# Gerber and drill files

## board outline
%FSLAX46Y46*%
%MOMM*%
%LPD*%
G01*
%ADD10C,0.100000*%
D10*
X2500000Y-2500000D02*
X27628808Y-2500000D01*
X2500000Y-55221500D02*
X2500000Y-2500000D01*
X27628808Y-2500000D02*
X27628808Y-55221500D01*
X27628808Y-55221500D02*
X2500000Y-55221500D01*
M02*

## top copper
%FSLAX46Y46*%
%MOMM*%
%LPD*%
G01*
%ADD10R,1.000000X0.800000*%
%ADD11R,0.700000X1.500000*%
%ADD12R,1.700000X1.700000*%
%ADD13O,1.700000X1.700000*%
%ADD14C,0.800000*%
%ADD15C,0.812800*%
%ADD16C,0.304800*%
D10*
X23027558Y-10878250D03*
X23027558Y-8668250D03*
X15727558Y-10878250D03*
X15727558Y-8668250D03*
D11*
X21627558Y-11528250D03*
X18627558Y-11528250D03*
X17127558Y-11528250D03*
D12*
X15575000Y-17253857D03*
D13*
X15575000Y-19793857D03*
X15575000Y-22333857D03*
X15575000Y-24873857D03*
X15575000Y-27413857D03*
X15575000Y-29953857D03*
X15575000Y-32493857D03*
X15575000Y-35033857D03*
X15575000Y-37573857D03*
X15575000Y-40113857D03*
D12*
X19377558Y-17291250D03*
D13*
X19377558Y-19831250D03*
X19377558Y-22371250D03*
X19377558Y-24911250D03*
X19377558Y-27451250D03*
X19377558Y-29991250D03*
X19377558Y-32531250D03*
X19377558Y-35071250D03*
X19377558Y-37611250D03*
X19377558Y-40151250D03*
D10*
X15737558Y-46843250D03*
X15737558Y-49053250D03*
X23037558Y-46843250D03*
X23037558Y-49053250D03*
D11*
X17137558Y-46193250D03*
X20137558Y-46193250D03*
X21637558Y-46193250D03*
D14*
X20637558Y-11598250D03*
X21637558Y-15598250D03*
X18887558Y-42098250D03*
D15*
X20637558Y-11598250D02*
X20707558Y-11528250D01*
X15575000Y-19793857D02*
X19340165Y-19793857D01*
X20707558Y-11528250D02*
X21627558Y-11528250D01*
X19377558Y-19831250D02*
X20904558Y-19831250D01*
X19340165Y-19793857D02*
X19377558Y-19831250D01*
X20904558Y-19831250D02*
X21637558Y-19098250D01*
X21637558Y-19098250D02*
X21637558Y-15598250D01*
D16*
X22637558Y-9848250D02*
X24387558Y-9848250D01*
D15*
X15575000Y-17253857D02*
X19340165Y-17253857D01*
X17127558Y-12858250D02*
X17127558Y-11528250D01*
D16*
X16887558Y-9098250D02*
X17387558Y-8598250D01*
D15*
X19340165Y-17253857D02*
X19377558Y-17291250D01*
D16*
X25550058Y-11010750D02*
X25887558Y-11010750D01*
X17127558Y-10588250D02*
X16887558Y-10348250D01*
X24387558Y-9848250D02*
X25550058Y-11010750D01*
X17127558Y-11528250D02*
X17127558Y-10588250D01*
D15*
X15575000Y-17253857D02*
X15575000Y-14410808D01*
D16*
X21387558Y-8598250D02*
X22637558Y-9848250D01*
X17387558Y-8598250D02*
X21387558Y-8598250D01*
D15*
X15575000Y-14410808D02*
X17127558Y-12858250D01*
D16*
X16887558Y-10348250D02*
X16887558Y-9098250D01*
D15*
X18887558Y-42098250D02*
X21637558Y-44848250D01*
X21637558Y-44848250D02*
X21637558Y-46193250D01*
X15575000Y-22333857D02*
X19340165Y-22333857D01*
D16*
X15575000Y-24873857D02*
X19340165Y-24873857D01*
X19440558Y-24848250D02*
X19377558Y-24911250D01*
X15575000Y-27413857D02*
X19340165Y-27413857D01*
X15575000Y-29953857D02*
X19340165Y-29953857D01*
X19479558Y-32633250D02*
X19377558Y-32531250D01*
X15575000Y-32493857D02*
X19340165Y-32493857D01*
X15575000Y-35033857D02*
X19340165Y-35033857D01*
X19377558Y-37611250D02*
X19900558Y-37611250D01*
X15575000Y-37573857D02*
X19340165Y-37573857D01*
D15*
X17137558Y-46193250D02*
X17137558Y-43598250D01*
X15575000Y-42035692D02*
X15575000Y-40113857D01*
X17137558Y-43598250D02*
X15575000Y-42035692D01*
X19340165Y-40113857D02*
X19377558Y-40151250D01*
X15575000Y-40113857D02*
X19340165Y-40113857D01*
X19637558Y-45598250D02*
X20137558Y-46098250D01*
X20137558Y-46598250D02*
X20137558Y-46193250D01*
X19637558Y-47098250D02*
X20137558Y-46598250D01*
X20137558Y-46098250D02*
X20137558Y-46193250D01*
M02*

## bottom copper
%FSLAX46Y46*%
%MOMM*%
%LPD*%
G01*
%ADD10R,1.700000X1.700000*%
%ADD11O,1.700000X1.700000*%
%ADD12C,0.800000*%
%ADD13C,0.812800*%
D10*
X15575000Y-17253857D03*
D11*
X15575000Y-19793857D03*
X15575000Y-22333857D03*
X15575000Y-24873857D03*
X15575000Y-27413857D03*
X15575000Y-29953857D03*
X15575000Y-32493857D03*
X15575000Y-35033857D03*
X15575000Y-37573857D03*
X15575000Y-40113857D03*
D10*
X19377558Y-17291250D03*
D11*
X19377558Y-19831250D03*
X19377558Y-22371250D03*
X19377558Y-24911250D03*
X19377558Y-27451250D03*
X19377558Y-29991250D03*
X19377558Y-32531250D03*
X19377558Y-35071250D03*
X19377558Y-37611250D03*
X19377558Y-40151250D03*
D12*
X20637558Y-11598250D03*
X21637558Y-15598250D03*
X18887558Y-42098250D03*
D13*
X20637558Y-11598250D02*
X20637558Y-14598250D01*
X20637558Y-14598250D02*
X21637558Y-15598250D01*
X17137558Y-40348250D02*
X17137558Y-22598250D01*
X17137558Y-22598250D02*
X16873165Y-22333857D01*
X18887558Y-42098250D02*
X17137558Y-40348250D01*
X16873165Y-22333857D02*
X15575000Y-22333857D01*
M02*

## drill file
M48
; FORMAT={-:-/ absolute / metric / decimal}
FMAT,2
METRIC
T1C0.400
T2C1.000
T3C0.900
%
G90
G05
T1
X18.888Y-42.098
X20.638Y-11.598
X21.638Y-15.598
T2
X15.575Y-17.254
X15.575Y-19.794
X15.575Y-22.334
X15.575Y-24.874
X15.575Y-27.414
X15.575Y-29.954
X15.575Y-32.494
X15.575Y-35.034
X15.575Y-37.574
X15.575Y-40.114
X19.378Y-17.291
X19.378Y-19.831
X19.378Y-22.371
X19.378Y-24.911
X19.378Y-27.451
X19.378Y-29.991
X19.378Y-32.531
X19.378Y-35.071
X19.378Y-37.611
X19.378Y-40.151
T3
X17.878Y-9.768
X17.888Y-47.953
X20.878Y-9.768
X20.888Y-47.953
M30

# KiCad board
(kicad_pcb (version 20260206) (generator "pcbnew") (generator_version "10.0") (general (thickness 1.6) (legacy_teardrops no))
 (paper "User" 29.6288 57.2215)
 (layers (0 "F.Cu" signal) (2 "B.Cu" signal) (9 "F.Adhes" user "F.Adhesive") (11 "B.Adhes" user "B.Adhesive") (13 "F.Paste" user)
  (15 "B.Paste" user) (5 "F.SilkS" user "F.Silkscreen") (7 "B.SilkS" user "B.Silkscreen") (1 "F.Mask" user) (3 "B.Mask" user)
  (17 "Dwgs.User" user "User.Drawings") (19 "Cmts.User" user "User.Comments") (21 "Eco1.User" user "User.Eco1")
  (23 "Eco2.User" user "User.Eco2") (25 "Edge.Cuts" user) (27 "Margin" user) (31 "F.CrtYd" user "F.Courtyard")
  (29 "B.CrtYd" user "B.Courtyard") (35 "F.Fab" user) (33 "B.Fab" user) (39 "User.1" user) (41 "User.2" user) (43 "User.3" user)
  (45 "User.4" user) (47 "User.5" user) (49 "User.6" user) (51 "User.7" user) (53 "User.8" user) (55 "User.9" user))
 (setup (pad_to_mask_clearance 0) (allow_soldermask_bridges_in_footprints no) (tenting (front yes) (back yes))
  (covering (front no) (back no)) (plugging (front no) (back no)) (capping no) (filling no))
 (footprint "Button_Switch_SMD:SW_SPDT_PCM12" (layer "F.Cu") (at 19.377558 10.09825 180)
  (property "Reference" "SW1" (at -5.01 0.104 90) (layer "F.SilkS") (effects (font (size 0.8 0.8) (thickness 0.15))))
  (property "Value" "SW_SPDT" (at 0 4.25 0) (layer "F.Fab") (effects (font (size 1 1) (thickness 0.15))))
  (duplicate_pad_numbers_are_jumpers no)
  (pad "" smd rect (at -3.65 -0.78 180) (size 1 0.8) (layers "F.Cu" "F.Mask" "F.Paste"))
  (pad "" smd rect (at -3.65 1.43 180) (size 1 0.8) (layers "F.Cu" "F.Mask" "F.Paste"))
  (pad "" np_thru_hole circle (at -1.5 0.33 180) (size 0.9 0.9) (drill 0.9) (layers "*.Cu" "*.Mask"))
  (pad "" np_thru_hole circle (at 1.5 0.33 180) (size 0.9 0.9) (drill 0.9) (layers "*.Cu" "*.Mask"))
  (pad "" smd rect (at 3.65 -0.78 180) (size 1 0.8) (layers "F.Cu" "F.Mask" "F.Paste"))
  (pad "" smd rect (at 3.65 1.43 180) (size 1 0.8) (layers "F.Cu" "F.Mask" "F.Paste"))
  (pad "1" smd rect (at -2.25 -1.43 180) (size 0.7 1.5) (layers "F.Cu" "F.Mask" "F.Paste") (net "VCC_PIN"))
  (pad "2" smd rect (at 0.75 -1.43 180) (size 0.7 1.5) (layers "F.Cu" "F.Mask" "F.Paste") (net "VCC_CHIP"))
  (pad "3" smd rect (at 2.25 -1.43 180) (size 0.7 1.5) (layers "F.Cu" "F.Mask" "F.Paste") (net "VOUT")))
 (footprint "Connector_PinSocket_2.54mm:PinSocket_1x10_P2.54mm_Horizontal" (layer "F.Cu") (at 15.575 17.253857)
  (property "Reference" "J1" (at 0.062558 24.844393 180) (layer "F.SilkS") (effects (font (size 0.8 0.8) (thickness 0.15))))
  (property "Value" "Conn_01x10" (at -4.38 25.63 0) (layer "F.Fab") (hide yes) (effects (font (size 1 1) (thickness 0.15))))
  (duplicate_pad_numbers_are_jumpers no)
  (pad "1" thru_hole rect (at 0 0) (size 1.7 1.7) (drill 1) (layers "*.Cu" "*.Mask") (remove_unused_layers no) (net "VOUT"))
  (pad "2" thru_hole oval (at 0 2.54) (size 1.7 1.7) (drill 1) (layers "*.Cu" "*.Mask") (remove_unused_layers no) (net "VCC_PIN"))
  (pad "3" thru_hole oval (at 0 5.08) (size 1.7 1.7) (drill 1) (layers "*.Cu" "*.Mask") (remove_unused_layers no) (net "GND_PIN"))
  (pad "4" thru_hole oval (at 0 7.62) (size 1.7 1.7) (drill 1) (layers "*.Cu" "*.Mask") (remove_unused_layers no) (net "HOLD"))
  (pad "5" thru_hole oval (at 0 10.16) (size 1.7 1.7) (drill 1) (layers "*.Cu" "*.Mask") (remove_unused_layers no) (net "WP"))
  (pad "6" thru_hole oval (at 0 12.7) (size 1.7 1.7) (drill 1) (layers "*.Cu" "*.Mask") (remove_unused_layers no) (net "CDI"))
  (pad "7" thru_hole oval (at 0 15.24) (size 1.7 1.7) (drill 1) (layers "*.Cu" "*.Mask") (remove_unused_layers no) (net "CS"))
  (pad "8" thru_hole oval (at 0 17.78) (size 1.7 1.7) (drill 1) (layers "*.Cu" "*.Mask") (remove_unused_layers no) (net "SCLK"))
  (pad "9" thru_hole oval (at 0 20.32) (size 1.7 1.7) (drill 1) (layers "*.Cu" "*.Mask") (remove_unused_layers no) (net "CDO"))
  (pad "10" thru_hole oval (at 0 22.86) (size 1.7 1.7) (drill 1) (layers "*.Cu" "*.Mask") (remove_unused_layers no) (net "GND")))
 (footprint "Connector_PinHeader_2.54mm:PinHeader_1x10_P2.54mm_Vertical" (layer "F.Cu") (at 19.377558 17.29125)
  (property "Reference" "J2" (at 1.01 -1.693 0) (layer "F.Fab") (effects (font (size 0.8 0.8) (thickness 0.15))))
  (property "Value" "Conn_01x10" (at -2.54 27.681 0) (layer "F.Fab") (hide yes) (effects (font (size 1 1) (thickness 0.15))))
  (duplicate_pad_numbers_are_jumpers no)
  (pad "1" thru_hole rect (at 0 0) (size 1.7 1.7) (drill 1) (layers "*.Cu" "*.Mask") (remove_unused_layers no) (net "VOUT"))
  (pad "2" thru_hole oval (at 0 2.54) (size 1.7 1.7) (drill 1) (layers "*.Cu" "*.Mask") (remove_unused_layers no) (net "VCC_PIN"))
  (pad "3" thru_hole oval (at 0 5.08) (size 1.7 1.7) (drill 1) (layers "*.Cu" "*.Mask") (remove_unused_layers no) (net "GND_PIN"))
  (pad "4" thru_hole oval (at 0 7.62) (size 1.7 1.7) (drill 1) (layers "*.Cu" "*.Mask") (remove_unused_layers no) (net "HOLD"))
  (pad "5" thru_hole oval (at 0 10.16) (size 1.7 1.7) (drill 1) (layers "*.Cu" "*.Mask") (remove_unused_layers no) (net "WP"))
  (pad "6" thru_hole oval (at 0 12.7) (size 1.7 1.7) (drill 1) (layers "*.Cu" "*.Mask") (remove_unused_layers no) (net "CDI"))
  (pad "7" thru_hole oval (at 0 15.24) (size 1.7 1.7) (drill 1) (layers "*.Cu" "*.Mask") (remove_unused_layers no) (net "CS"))
  (pad "8" thru_hole oval (at 0 17.78) (size 1.7 1.7) (drill 1) (layers "*.Cu" "*.Mask") (remove_unused_layers no) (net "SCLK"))
  (pad "9" thru_hole oval (at 0 20.32) (size 1.7 1.7) (drill 1) (layers "*.Cu" "*.Mask") (remove_unused_layers no) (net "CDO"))
  (pad "10" thru_hole oval (at 0 22.86) (size 1.7 1.7) (drill 1) (layers "*.Cu" "*.Mask") (remove_unused_layers no) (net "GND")))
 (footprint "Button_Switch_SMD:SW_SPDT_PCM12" (layer "F.Cu") (at 19.387558 47.62325)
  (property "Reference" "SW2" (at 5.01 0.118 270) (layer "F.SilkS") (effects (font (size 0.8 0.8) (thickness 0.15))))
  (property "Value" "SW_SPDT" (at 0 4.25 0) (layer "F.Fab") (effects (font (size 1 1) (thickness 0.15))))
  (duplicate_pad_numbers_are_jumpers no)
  (pad "" smd rect (at -3.65 -0.78) (size 1 0.8) (layers "F.Cu" "F.Mask" "F.Paste"))
  (pad "" smd rect (at -3.65 1.43) (size 1 0.8) (layers "F.Cu" "F.Mask" "F.Paste"))
  (pad "" np_thru_hole circle (at -1.5 0.33) (size 0.9 0.9) (drill 0.9) (layers "*.Cu" "*.Mask"))
  (pad "" np_thru_hole circle (at 1.5 0.33) (size 0.9 0.9) (drill 0.9) (layers "*.Cu" "*.Mask"))
  (pad "" smd rect (at 3.65 -0.78) (size 1 0.8) (layers "F.Cu" "F.Mask" "F.Paste"))
  (pad "" smd rect (at 3.65 1.43) (size 1 0.8) (layers "F.Cu" "F.Mask" "F.Paste"))
  (pad "1" smd rect (at -2.25 -1.43) (size 0.7 1.5) (layers "F.Cu" "F.Mask" "F.Paste") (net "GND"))
  (pad "2" smd rect (at 0.75 -1.43) (size 0.7 1.5) (layers "F.Cu" "F.Mask" "F.Paste") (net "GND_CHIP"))
  (pad "3" smd rect (at 2.25 -1.43) (size 0.7 1.5) (layers "F.Cu" "F.Mask" "F.Paste") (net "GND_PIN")))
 (gr_line (start 2.5 2.5) (end 27.628808 2.5) (stroke (width 0.1) (type default)) (layer "Edge.Cuts"))
 (gr_line (start 2.5 55.2215) (end 2.5 2.5) (stroke (width 0.1) (type default)) (layer "Edge.Cuts"))
 (gr_line (start 27.628808 2.5) (end 27.628808 55.2215) (stroke (width 0.1) (type default)) (layer "Edge.Cuts"))
 (gr_line (start 27.628808 55.2215) (end 2.5 55.2215) (stroke (width 0.1) (type default)) (layer "Edge.Cuts"))
 (segment (start 20.637558 11.59825) (end 20.707558 11.52825) (width 0.8128) (layer "F.Cu") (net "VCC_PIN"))
 (segment (start 15.575 19.793857) (end 19.340165 19.793857) (width 0.8128) (layer "F.Cu") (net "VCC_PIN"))
 (segment (start 20.707558 11.52825) (end 21.627558 11.52825) (width 0.8128) (layer "F.Cu") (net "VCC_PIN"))
 (segment (start 19.377558 19.83125) (end 20.904558 19.83125) (width 0.8128) (layer "F.Cu") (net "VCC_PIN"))
 (segment (start 19.340165 19.793857) (end 19.377558 19.83125) (width 0.8128) (layer "F.Cu") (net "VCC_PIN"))
 (segment (start 20.904558 19.83125) (end 21.637558 19.09825) (width 0.8128) (layer "F.Cu") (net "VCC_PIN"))
 (segment (start 21.637558 19.09825) (end 21.637558 15.59825) (width 0.8128) (layer "F.Cu") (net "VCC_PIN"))
 (via (at 20.637558 11.59825) (size 0.8) (drill 0.4) (layers "F.Cu" "B.Cu") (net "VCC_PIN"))
 (via (at 21.637558 15.59825) (size 0.8) (drill 0.4) (layers "F.Cu" "B.Cu") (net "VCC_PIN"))
 (segment (start 20.637558 11.59825) (end 20.637558 14.59825) (width 0.8128) (layer "B.Cu") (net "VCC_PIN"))
 (segment (start 20.637558 14.59825) (end 21.637558 15.59825) (width 0.8128) (layer "B.Cu") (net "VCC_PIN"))
 (segment (start 22.637558 9.84825) (end 24.387558 9.84825) (width 0.3048) (layer "F.Cu") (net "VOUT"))
 (segment (start 15.575 17.253857) (end 19.340165 17.253857) (width 0.8128) (layer "F.Cu") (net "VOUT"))
 (segment (start 17.127558 12.85825) (end 17.127558 11.52825) (width 0.8128) (layer "F.Cu") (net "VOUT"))
 (segment (start 16.887558 9.09825) (end 17.387558 8.59825) (width 0.3048) (layer "F.Cu") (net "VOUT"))
 (segment (start 19.340165 17.253857) (end 19.377558 17.29125) (width 0.8128) (layer "F.Cu") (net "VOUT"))
 (segment (start 25.550058 11.01075) (end 25.887558 11.01075) (width 0.3048) (layer "F.Cu") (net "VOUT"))
 (segment (start 17.127558 10.58825) (end 16.887558 10.34825) (width 0.3048) (layer "F.Cu") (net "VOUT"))
 (segment (start 24.387558 9.84825) (end 25.550058 11.01075) (width 0.3048) (layer "F.Cu") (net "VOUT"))
 (segment (start 17.127558 11.52825) (end 17.127558 10.58825) (width 0.3048) (layer "F.Cu") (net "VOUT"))
 (segment (start 15.575 17.253857) (end 15.575 14.410808) (width 0.8128) (layer "F.Cu") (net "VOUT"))
 (segment (start 21.387558 8.59825) (end 22.637558 9.84825) (width 0.3048) (layer "F.Cu") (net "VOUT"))
 (segment (start 17.387558 8.59825) (end 21.387558 8.59825) (width 0.3048) (layer "F.Cu") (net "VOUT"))
 (segment (start 15.575 14.410808) (end 17.127558 12.85825) (width 0.8128) (layer "F.Cu") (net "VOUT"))
 (segment (start 16.887558 10.34825) (end 16.887558 9.09825) (width 0.3048) (layer "F.Cu") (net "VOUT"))
 (segment (start 18.887558 42.09825) (end 21.637558 44.84825) (width 0.8128) (layer "F.Cu") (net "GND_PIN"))
 (segment (start 21.637558 44.84825) (end 21.637558 46.19325) (width 0.8128) (layer "F.Cu") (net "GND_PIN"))
 (segment (start 15.575 22.333857) (end 19.340165 22.333857) (width 0.8128) (layer "F.Cu") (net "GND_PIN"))
 (via (at 18.887558 42.09825) (size 0.8) (drill 0.4) (layers "F.Cu" "B.Cu") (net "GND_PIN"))
 (segment (start 17.137558 40.34825) (end 17.137558 22.59825) (width 0.8128) (layer "B.Cu") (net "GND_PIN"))
 (segment (start 17.137558 22.59825) (end 16.873165 22.333857) (width 0.8128) (layer "B.Cu") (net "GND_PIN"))
 (segment (start 18.887558 42.09825) (end 17.137558 40.34825) (width 0.8128) (layer "B.Cu") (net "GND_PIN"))
 (segment (start 16.873165 22.333857) (end 15.575 22.333857) (width 0.8128) (layer "B.Cu") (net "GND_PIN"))
 (segment (start 15.575 24.873857) (end 19.340165 24.873857) (width 0.3048) (layer "F.Cu") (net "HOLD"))
 (segment (start 19.440558 24.84825) (end 19.377558 24.91125) (width 0.3048) (layer "F.Cu") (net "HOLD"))
 (segment (start 15.575 27.413857) (end 19.340165 27.413857) (width 0.3048) (layer "F.Cu") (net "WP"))
 (segment (start 15.575 29.953857) (end 19.340165 29.953857) (width 0.3048) (layer "F.Cu") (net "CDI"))
 (segment (start 19.479558 32.63325) (end 19.377558 32.53125) (width 0.3048) (layer "F.Cu") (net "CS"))
 (segment (start 15.575 32.493857) (end 19.340165 32.493857) (width 0.3048) (layer "F.Cu") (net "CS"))
 (segment (start 15.575 35.033857) (end 19.340165 35.033857) (width 0.3048) (layer "F.Cu") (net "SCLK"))
 (segment (start 19.377558 37.61125) (end 19.900558 37.61125) (width 0.3048) (layer "F.Cu") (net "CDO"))
 (segment (start 15.575 37.573857) (end 19.340165 37.573857) (width 0.3048) (layer "F.Cu") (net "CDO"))
 (segment (start 17.137558 46.19325) (end 17.137558 43.59825) (width 0.8128) (layer "F.Cu") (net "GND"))
 (segment (start 15.575 42.035692) (end 15.575 40.113857) (width 0.8128) (layer "F.Cu") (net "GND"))
 (segment (start 17.137558 43.59825) (end 15.575 42.035692) (width 0.8128) (layer "F.Cu") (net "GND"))
 (segment (start 19.340165 40.113857) (end 19.377558 40.15125) (width 0.8128) (layer "F.Cu") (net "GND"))
 (segment (start 15.575 40.113857) (end 19.340165 40.113857) (width 0.8128) (layer "F.Cu") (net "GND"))
 (segment (start 19.637558 45.59825) (end 20.137558 46.09825) (width 0.8128) (layer "F.Cu") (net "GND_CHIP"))
 (segment (start 20.137558 46.59825) (end 20.137558 46.19325) (width 0.8128) (layer "F.Cu") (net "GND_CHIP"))
 (segment (start 19.637558 47.09825) (end 20.137558 46.59825) (width 0.8128) (layer "F.Cu") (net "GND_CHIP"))
 (segment (start 20.137558 46.09825) (end 20.137558 46.19325) (width 0.8128) (layer "F.Cu") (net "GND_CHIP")))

